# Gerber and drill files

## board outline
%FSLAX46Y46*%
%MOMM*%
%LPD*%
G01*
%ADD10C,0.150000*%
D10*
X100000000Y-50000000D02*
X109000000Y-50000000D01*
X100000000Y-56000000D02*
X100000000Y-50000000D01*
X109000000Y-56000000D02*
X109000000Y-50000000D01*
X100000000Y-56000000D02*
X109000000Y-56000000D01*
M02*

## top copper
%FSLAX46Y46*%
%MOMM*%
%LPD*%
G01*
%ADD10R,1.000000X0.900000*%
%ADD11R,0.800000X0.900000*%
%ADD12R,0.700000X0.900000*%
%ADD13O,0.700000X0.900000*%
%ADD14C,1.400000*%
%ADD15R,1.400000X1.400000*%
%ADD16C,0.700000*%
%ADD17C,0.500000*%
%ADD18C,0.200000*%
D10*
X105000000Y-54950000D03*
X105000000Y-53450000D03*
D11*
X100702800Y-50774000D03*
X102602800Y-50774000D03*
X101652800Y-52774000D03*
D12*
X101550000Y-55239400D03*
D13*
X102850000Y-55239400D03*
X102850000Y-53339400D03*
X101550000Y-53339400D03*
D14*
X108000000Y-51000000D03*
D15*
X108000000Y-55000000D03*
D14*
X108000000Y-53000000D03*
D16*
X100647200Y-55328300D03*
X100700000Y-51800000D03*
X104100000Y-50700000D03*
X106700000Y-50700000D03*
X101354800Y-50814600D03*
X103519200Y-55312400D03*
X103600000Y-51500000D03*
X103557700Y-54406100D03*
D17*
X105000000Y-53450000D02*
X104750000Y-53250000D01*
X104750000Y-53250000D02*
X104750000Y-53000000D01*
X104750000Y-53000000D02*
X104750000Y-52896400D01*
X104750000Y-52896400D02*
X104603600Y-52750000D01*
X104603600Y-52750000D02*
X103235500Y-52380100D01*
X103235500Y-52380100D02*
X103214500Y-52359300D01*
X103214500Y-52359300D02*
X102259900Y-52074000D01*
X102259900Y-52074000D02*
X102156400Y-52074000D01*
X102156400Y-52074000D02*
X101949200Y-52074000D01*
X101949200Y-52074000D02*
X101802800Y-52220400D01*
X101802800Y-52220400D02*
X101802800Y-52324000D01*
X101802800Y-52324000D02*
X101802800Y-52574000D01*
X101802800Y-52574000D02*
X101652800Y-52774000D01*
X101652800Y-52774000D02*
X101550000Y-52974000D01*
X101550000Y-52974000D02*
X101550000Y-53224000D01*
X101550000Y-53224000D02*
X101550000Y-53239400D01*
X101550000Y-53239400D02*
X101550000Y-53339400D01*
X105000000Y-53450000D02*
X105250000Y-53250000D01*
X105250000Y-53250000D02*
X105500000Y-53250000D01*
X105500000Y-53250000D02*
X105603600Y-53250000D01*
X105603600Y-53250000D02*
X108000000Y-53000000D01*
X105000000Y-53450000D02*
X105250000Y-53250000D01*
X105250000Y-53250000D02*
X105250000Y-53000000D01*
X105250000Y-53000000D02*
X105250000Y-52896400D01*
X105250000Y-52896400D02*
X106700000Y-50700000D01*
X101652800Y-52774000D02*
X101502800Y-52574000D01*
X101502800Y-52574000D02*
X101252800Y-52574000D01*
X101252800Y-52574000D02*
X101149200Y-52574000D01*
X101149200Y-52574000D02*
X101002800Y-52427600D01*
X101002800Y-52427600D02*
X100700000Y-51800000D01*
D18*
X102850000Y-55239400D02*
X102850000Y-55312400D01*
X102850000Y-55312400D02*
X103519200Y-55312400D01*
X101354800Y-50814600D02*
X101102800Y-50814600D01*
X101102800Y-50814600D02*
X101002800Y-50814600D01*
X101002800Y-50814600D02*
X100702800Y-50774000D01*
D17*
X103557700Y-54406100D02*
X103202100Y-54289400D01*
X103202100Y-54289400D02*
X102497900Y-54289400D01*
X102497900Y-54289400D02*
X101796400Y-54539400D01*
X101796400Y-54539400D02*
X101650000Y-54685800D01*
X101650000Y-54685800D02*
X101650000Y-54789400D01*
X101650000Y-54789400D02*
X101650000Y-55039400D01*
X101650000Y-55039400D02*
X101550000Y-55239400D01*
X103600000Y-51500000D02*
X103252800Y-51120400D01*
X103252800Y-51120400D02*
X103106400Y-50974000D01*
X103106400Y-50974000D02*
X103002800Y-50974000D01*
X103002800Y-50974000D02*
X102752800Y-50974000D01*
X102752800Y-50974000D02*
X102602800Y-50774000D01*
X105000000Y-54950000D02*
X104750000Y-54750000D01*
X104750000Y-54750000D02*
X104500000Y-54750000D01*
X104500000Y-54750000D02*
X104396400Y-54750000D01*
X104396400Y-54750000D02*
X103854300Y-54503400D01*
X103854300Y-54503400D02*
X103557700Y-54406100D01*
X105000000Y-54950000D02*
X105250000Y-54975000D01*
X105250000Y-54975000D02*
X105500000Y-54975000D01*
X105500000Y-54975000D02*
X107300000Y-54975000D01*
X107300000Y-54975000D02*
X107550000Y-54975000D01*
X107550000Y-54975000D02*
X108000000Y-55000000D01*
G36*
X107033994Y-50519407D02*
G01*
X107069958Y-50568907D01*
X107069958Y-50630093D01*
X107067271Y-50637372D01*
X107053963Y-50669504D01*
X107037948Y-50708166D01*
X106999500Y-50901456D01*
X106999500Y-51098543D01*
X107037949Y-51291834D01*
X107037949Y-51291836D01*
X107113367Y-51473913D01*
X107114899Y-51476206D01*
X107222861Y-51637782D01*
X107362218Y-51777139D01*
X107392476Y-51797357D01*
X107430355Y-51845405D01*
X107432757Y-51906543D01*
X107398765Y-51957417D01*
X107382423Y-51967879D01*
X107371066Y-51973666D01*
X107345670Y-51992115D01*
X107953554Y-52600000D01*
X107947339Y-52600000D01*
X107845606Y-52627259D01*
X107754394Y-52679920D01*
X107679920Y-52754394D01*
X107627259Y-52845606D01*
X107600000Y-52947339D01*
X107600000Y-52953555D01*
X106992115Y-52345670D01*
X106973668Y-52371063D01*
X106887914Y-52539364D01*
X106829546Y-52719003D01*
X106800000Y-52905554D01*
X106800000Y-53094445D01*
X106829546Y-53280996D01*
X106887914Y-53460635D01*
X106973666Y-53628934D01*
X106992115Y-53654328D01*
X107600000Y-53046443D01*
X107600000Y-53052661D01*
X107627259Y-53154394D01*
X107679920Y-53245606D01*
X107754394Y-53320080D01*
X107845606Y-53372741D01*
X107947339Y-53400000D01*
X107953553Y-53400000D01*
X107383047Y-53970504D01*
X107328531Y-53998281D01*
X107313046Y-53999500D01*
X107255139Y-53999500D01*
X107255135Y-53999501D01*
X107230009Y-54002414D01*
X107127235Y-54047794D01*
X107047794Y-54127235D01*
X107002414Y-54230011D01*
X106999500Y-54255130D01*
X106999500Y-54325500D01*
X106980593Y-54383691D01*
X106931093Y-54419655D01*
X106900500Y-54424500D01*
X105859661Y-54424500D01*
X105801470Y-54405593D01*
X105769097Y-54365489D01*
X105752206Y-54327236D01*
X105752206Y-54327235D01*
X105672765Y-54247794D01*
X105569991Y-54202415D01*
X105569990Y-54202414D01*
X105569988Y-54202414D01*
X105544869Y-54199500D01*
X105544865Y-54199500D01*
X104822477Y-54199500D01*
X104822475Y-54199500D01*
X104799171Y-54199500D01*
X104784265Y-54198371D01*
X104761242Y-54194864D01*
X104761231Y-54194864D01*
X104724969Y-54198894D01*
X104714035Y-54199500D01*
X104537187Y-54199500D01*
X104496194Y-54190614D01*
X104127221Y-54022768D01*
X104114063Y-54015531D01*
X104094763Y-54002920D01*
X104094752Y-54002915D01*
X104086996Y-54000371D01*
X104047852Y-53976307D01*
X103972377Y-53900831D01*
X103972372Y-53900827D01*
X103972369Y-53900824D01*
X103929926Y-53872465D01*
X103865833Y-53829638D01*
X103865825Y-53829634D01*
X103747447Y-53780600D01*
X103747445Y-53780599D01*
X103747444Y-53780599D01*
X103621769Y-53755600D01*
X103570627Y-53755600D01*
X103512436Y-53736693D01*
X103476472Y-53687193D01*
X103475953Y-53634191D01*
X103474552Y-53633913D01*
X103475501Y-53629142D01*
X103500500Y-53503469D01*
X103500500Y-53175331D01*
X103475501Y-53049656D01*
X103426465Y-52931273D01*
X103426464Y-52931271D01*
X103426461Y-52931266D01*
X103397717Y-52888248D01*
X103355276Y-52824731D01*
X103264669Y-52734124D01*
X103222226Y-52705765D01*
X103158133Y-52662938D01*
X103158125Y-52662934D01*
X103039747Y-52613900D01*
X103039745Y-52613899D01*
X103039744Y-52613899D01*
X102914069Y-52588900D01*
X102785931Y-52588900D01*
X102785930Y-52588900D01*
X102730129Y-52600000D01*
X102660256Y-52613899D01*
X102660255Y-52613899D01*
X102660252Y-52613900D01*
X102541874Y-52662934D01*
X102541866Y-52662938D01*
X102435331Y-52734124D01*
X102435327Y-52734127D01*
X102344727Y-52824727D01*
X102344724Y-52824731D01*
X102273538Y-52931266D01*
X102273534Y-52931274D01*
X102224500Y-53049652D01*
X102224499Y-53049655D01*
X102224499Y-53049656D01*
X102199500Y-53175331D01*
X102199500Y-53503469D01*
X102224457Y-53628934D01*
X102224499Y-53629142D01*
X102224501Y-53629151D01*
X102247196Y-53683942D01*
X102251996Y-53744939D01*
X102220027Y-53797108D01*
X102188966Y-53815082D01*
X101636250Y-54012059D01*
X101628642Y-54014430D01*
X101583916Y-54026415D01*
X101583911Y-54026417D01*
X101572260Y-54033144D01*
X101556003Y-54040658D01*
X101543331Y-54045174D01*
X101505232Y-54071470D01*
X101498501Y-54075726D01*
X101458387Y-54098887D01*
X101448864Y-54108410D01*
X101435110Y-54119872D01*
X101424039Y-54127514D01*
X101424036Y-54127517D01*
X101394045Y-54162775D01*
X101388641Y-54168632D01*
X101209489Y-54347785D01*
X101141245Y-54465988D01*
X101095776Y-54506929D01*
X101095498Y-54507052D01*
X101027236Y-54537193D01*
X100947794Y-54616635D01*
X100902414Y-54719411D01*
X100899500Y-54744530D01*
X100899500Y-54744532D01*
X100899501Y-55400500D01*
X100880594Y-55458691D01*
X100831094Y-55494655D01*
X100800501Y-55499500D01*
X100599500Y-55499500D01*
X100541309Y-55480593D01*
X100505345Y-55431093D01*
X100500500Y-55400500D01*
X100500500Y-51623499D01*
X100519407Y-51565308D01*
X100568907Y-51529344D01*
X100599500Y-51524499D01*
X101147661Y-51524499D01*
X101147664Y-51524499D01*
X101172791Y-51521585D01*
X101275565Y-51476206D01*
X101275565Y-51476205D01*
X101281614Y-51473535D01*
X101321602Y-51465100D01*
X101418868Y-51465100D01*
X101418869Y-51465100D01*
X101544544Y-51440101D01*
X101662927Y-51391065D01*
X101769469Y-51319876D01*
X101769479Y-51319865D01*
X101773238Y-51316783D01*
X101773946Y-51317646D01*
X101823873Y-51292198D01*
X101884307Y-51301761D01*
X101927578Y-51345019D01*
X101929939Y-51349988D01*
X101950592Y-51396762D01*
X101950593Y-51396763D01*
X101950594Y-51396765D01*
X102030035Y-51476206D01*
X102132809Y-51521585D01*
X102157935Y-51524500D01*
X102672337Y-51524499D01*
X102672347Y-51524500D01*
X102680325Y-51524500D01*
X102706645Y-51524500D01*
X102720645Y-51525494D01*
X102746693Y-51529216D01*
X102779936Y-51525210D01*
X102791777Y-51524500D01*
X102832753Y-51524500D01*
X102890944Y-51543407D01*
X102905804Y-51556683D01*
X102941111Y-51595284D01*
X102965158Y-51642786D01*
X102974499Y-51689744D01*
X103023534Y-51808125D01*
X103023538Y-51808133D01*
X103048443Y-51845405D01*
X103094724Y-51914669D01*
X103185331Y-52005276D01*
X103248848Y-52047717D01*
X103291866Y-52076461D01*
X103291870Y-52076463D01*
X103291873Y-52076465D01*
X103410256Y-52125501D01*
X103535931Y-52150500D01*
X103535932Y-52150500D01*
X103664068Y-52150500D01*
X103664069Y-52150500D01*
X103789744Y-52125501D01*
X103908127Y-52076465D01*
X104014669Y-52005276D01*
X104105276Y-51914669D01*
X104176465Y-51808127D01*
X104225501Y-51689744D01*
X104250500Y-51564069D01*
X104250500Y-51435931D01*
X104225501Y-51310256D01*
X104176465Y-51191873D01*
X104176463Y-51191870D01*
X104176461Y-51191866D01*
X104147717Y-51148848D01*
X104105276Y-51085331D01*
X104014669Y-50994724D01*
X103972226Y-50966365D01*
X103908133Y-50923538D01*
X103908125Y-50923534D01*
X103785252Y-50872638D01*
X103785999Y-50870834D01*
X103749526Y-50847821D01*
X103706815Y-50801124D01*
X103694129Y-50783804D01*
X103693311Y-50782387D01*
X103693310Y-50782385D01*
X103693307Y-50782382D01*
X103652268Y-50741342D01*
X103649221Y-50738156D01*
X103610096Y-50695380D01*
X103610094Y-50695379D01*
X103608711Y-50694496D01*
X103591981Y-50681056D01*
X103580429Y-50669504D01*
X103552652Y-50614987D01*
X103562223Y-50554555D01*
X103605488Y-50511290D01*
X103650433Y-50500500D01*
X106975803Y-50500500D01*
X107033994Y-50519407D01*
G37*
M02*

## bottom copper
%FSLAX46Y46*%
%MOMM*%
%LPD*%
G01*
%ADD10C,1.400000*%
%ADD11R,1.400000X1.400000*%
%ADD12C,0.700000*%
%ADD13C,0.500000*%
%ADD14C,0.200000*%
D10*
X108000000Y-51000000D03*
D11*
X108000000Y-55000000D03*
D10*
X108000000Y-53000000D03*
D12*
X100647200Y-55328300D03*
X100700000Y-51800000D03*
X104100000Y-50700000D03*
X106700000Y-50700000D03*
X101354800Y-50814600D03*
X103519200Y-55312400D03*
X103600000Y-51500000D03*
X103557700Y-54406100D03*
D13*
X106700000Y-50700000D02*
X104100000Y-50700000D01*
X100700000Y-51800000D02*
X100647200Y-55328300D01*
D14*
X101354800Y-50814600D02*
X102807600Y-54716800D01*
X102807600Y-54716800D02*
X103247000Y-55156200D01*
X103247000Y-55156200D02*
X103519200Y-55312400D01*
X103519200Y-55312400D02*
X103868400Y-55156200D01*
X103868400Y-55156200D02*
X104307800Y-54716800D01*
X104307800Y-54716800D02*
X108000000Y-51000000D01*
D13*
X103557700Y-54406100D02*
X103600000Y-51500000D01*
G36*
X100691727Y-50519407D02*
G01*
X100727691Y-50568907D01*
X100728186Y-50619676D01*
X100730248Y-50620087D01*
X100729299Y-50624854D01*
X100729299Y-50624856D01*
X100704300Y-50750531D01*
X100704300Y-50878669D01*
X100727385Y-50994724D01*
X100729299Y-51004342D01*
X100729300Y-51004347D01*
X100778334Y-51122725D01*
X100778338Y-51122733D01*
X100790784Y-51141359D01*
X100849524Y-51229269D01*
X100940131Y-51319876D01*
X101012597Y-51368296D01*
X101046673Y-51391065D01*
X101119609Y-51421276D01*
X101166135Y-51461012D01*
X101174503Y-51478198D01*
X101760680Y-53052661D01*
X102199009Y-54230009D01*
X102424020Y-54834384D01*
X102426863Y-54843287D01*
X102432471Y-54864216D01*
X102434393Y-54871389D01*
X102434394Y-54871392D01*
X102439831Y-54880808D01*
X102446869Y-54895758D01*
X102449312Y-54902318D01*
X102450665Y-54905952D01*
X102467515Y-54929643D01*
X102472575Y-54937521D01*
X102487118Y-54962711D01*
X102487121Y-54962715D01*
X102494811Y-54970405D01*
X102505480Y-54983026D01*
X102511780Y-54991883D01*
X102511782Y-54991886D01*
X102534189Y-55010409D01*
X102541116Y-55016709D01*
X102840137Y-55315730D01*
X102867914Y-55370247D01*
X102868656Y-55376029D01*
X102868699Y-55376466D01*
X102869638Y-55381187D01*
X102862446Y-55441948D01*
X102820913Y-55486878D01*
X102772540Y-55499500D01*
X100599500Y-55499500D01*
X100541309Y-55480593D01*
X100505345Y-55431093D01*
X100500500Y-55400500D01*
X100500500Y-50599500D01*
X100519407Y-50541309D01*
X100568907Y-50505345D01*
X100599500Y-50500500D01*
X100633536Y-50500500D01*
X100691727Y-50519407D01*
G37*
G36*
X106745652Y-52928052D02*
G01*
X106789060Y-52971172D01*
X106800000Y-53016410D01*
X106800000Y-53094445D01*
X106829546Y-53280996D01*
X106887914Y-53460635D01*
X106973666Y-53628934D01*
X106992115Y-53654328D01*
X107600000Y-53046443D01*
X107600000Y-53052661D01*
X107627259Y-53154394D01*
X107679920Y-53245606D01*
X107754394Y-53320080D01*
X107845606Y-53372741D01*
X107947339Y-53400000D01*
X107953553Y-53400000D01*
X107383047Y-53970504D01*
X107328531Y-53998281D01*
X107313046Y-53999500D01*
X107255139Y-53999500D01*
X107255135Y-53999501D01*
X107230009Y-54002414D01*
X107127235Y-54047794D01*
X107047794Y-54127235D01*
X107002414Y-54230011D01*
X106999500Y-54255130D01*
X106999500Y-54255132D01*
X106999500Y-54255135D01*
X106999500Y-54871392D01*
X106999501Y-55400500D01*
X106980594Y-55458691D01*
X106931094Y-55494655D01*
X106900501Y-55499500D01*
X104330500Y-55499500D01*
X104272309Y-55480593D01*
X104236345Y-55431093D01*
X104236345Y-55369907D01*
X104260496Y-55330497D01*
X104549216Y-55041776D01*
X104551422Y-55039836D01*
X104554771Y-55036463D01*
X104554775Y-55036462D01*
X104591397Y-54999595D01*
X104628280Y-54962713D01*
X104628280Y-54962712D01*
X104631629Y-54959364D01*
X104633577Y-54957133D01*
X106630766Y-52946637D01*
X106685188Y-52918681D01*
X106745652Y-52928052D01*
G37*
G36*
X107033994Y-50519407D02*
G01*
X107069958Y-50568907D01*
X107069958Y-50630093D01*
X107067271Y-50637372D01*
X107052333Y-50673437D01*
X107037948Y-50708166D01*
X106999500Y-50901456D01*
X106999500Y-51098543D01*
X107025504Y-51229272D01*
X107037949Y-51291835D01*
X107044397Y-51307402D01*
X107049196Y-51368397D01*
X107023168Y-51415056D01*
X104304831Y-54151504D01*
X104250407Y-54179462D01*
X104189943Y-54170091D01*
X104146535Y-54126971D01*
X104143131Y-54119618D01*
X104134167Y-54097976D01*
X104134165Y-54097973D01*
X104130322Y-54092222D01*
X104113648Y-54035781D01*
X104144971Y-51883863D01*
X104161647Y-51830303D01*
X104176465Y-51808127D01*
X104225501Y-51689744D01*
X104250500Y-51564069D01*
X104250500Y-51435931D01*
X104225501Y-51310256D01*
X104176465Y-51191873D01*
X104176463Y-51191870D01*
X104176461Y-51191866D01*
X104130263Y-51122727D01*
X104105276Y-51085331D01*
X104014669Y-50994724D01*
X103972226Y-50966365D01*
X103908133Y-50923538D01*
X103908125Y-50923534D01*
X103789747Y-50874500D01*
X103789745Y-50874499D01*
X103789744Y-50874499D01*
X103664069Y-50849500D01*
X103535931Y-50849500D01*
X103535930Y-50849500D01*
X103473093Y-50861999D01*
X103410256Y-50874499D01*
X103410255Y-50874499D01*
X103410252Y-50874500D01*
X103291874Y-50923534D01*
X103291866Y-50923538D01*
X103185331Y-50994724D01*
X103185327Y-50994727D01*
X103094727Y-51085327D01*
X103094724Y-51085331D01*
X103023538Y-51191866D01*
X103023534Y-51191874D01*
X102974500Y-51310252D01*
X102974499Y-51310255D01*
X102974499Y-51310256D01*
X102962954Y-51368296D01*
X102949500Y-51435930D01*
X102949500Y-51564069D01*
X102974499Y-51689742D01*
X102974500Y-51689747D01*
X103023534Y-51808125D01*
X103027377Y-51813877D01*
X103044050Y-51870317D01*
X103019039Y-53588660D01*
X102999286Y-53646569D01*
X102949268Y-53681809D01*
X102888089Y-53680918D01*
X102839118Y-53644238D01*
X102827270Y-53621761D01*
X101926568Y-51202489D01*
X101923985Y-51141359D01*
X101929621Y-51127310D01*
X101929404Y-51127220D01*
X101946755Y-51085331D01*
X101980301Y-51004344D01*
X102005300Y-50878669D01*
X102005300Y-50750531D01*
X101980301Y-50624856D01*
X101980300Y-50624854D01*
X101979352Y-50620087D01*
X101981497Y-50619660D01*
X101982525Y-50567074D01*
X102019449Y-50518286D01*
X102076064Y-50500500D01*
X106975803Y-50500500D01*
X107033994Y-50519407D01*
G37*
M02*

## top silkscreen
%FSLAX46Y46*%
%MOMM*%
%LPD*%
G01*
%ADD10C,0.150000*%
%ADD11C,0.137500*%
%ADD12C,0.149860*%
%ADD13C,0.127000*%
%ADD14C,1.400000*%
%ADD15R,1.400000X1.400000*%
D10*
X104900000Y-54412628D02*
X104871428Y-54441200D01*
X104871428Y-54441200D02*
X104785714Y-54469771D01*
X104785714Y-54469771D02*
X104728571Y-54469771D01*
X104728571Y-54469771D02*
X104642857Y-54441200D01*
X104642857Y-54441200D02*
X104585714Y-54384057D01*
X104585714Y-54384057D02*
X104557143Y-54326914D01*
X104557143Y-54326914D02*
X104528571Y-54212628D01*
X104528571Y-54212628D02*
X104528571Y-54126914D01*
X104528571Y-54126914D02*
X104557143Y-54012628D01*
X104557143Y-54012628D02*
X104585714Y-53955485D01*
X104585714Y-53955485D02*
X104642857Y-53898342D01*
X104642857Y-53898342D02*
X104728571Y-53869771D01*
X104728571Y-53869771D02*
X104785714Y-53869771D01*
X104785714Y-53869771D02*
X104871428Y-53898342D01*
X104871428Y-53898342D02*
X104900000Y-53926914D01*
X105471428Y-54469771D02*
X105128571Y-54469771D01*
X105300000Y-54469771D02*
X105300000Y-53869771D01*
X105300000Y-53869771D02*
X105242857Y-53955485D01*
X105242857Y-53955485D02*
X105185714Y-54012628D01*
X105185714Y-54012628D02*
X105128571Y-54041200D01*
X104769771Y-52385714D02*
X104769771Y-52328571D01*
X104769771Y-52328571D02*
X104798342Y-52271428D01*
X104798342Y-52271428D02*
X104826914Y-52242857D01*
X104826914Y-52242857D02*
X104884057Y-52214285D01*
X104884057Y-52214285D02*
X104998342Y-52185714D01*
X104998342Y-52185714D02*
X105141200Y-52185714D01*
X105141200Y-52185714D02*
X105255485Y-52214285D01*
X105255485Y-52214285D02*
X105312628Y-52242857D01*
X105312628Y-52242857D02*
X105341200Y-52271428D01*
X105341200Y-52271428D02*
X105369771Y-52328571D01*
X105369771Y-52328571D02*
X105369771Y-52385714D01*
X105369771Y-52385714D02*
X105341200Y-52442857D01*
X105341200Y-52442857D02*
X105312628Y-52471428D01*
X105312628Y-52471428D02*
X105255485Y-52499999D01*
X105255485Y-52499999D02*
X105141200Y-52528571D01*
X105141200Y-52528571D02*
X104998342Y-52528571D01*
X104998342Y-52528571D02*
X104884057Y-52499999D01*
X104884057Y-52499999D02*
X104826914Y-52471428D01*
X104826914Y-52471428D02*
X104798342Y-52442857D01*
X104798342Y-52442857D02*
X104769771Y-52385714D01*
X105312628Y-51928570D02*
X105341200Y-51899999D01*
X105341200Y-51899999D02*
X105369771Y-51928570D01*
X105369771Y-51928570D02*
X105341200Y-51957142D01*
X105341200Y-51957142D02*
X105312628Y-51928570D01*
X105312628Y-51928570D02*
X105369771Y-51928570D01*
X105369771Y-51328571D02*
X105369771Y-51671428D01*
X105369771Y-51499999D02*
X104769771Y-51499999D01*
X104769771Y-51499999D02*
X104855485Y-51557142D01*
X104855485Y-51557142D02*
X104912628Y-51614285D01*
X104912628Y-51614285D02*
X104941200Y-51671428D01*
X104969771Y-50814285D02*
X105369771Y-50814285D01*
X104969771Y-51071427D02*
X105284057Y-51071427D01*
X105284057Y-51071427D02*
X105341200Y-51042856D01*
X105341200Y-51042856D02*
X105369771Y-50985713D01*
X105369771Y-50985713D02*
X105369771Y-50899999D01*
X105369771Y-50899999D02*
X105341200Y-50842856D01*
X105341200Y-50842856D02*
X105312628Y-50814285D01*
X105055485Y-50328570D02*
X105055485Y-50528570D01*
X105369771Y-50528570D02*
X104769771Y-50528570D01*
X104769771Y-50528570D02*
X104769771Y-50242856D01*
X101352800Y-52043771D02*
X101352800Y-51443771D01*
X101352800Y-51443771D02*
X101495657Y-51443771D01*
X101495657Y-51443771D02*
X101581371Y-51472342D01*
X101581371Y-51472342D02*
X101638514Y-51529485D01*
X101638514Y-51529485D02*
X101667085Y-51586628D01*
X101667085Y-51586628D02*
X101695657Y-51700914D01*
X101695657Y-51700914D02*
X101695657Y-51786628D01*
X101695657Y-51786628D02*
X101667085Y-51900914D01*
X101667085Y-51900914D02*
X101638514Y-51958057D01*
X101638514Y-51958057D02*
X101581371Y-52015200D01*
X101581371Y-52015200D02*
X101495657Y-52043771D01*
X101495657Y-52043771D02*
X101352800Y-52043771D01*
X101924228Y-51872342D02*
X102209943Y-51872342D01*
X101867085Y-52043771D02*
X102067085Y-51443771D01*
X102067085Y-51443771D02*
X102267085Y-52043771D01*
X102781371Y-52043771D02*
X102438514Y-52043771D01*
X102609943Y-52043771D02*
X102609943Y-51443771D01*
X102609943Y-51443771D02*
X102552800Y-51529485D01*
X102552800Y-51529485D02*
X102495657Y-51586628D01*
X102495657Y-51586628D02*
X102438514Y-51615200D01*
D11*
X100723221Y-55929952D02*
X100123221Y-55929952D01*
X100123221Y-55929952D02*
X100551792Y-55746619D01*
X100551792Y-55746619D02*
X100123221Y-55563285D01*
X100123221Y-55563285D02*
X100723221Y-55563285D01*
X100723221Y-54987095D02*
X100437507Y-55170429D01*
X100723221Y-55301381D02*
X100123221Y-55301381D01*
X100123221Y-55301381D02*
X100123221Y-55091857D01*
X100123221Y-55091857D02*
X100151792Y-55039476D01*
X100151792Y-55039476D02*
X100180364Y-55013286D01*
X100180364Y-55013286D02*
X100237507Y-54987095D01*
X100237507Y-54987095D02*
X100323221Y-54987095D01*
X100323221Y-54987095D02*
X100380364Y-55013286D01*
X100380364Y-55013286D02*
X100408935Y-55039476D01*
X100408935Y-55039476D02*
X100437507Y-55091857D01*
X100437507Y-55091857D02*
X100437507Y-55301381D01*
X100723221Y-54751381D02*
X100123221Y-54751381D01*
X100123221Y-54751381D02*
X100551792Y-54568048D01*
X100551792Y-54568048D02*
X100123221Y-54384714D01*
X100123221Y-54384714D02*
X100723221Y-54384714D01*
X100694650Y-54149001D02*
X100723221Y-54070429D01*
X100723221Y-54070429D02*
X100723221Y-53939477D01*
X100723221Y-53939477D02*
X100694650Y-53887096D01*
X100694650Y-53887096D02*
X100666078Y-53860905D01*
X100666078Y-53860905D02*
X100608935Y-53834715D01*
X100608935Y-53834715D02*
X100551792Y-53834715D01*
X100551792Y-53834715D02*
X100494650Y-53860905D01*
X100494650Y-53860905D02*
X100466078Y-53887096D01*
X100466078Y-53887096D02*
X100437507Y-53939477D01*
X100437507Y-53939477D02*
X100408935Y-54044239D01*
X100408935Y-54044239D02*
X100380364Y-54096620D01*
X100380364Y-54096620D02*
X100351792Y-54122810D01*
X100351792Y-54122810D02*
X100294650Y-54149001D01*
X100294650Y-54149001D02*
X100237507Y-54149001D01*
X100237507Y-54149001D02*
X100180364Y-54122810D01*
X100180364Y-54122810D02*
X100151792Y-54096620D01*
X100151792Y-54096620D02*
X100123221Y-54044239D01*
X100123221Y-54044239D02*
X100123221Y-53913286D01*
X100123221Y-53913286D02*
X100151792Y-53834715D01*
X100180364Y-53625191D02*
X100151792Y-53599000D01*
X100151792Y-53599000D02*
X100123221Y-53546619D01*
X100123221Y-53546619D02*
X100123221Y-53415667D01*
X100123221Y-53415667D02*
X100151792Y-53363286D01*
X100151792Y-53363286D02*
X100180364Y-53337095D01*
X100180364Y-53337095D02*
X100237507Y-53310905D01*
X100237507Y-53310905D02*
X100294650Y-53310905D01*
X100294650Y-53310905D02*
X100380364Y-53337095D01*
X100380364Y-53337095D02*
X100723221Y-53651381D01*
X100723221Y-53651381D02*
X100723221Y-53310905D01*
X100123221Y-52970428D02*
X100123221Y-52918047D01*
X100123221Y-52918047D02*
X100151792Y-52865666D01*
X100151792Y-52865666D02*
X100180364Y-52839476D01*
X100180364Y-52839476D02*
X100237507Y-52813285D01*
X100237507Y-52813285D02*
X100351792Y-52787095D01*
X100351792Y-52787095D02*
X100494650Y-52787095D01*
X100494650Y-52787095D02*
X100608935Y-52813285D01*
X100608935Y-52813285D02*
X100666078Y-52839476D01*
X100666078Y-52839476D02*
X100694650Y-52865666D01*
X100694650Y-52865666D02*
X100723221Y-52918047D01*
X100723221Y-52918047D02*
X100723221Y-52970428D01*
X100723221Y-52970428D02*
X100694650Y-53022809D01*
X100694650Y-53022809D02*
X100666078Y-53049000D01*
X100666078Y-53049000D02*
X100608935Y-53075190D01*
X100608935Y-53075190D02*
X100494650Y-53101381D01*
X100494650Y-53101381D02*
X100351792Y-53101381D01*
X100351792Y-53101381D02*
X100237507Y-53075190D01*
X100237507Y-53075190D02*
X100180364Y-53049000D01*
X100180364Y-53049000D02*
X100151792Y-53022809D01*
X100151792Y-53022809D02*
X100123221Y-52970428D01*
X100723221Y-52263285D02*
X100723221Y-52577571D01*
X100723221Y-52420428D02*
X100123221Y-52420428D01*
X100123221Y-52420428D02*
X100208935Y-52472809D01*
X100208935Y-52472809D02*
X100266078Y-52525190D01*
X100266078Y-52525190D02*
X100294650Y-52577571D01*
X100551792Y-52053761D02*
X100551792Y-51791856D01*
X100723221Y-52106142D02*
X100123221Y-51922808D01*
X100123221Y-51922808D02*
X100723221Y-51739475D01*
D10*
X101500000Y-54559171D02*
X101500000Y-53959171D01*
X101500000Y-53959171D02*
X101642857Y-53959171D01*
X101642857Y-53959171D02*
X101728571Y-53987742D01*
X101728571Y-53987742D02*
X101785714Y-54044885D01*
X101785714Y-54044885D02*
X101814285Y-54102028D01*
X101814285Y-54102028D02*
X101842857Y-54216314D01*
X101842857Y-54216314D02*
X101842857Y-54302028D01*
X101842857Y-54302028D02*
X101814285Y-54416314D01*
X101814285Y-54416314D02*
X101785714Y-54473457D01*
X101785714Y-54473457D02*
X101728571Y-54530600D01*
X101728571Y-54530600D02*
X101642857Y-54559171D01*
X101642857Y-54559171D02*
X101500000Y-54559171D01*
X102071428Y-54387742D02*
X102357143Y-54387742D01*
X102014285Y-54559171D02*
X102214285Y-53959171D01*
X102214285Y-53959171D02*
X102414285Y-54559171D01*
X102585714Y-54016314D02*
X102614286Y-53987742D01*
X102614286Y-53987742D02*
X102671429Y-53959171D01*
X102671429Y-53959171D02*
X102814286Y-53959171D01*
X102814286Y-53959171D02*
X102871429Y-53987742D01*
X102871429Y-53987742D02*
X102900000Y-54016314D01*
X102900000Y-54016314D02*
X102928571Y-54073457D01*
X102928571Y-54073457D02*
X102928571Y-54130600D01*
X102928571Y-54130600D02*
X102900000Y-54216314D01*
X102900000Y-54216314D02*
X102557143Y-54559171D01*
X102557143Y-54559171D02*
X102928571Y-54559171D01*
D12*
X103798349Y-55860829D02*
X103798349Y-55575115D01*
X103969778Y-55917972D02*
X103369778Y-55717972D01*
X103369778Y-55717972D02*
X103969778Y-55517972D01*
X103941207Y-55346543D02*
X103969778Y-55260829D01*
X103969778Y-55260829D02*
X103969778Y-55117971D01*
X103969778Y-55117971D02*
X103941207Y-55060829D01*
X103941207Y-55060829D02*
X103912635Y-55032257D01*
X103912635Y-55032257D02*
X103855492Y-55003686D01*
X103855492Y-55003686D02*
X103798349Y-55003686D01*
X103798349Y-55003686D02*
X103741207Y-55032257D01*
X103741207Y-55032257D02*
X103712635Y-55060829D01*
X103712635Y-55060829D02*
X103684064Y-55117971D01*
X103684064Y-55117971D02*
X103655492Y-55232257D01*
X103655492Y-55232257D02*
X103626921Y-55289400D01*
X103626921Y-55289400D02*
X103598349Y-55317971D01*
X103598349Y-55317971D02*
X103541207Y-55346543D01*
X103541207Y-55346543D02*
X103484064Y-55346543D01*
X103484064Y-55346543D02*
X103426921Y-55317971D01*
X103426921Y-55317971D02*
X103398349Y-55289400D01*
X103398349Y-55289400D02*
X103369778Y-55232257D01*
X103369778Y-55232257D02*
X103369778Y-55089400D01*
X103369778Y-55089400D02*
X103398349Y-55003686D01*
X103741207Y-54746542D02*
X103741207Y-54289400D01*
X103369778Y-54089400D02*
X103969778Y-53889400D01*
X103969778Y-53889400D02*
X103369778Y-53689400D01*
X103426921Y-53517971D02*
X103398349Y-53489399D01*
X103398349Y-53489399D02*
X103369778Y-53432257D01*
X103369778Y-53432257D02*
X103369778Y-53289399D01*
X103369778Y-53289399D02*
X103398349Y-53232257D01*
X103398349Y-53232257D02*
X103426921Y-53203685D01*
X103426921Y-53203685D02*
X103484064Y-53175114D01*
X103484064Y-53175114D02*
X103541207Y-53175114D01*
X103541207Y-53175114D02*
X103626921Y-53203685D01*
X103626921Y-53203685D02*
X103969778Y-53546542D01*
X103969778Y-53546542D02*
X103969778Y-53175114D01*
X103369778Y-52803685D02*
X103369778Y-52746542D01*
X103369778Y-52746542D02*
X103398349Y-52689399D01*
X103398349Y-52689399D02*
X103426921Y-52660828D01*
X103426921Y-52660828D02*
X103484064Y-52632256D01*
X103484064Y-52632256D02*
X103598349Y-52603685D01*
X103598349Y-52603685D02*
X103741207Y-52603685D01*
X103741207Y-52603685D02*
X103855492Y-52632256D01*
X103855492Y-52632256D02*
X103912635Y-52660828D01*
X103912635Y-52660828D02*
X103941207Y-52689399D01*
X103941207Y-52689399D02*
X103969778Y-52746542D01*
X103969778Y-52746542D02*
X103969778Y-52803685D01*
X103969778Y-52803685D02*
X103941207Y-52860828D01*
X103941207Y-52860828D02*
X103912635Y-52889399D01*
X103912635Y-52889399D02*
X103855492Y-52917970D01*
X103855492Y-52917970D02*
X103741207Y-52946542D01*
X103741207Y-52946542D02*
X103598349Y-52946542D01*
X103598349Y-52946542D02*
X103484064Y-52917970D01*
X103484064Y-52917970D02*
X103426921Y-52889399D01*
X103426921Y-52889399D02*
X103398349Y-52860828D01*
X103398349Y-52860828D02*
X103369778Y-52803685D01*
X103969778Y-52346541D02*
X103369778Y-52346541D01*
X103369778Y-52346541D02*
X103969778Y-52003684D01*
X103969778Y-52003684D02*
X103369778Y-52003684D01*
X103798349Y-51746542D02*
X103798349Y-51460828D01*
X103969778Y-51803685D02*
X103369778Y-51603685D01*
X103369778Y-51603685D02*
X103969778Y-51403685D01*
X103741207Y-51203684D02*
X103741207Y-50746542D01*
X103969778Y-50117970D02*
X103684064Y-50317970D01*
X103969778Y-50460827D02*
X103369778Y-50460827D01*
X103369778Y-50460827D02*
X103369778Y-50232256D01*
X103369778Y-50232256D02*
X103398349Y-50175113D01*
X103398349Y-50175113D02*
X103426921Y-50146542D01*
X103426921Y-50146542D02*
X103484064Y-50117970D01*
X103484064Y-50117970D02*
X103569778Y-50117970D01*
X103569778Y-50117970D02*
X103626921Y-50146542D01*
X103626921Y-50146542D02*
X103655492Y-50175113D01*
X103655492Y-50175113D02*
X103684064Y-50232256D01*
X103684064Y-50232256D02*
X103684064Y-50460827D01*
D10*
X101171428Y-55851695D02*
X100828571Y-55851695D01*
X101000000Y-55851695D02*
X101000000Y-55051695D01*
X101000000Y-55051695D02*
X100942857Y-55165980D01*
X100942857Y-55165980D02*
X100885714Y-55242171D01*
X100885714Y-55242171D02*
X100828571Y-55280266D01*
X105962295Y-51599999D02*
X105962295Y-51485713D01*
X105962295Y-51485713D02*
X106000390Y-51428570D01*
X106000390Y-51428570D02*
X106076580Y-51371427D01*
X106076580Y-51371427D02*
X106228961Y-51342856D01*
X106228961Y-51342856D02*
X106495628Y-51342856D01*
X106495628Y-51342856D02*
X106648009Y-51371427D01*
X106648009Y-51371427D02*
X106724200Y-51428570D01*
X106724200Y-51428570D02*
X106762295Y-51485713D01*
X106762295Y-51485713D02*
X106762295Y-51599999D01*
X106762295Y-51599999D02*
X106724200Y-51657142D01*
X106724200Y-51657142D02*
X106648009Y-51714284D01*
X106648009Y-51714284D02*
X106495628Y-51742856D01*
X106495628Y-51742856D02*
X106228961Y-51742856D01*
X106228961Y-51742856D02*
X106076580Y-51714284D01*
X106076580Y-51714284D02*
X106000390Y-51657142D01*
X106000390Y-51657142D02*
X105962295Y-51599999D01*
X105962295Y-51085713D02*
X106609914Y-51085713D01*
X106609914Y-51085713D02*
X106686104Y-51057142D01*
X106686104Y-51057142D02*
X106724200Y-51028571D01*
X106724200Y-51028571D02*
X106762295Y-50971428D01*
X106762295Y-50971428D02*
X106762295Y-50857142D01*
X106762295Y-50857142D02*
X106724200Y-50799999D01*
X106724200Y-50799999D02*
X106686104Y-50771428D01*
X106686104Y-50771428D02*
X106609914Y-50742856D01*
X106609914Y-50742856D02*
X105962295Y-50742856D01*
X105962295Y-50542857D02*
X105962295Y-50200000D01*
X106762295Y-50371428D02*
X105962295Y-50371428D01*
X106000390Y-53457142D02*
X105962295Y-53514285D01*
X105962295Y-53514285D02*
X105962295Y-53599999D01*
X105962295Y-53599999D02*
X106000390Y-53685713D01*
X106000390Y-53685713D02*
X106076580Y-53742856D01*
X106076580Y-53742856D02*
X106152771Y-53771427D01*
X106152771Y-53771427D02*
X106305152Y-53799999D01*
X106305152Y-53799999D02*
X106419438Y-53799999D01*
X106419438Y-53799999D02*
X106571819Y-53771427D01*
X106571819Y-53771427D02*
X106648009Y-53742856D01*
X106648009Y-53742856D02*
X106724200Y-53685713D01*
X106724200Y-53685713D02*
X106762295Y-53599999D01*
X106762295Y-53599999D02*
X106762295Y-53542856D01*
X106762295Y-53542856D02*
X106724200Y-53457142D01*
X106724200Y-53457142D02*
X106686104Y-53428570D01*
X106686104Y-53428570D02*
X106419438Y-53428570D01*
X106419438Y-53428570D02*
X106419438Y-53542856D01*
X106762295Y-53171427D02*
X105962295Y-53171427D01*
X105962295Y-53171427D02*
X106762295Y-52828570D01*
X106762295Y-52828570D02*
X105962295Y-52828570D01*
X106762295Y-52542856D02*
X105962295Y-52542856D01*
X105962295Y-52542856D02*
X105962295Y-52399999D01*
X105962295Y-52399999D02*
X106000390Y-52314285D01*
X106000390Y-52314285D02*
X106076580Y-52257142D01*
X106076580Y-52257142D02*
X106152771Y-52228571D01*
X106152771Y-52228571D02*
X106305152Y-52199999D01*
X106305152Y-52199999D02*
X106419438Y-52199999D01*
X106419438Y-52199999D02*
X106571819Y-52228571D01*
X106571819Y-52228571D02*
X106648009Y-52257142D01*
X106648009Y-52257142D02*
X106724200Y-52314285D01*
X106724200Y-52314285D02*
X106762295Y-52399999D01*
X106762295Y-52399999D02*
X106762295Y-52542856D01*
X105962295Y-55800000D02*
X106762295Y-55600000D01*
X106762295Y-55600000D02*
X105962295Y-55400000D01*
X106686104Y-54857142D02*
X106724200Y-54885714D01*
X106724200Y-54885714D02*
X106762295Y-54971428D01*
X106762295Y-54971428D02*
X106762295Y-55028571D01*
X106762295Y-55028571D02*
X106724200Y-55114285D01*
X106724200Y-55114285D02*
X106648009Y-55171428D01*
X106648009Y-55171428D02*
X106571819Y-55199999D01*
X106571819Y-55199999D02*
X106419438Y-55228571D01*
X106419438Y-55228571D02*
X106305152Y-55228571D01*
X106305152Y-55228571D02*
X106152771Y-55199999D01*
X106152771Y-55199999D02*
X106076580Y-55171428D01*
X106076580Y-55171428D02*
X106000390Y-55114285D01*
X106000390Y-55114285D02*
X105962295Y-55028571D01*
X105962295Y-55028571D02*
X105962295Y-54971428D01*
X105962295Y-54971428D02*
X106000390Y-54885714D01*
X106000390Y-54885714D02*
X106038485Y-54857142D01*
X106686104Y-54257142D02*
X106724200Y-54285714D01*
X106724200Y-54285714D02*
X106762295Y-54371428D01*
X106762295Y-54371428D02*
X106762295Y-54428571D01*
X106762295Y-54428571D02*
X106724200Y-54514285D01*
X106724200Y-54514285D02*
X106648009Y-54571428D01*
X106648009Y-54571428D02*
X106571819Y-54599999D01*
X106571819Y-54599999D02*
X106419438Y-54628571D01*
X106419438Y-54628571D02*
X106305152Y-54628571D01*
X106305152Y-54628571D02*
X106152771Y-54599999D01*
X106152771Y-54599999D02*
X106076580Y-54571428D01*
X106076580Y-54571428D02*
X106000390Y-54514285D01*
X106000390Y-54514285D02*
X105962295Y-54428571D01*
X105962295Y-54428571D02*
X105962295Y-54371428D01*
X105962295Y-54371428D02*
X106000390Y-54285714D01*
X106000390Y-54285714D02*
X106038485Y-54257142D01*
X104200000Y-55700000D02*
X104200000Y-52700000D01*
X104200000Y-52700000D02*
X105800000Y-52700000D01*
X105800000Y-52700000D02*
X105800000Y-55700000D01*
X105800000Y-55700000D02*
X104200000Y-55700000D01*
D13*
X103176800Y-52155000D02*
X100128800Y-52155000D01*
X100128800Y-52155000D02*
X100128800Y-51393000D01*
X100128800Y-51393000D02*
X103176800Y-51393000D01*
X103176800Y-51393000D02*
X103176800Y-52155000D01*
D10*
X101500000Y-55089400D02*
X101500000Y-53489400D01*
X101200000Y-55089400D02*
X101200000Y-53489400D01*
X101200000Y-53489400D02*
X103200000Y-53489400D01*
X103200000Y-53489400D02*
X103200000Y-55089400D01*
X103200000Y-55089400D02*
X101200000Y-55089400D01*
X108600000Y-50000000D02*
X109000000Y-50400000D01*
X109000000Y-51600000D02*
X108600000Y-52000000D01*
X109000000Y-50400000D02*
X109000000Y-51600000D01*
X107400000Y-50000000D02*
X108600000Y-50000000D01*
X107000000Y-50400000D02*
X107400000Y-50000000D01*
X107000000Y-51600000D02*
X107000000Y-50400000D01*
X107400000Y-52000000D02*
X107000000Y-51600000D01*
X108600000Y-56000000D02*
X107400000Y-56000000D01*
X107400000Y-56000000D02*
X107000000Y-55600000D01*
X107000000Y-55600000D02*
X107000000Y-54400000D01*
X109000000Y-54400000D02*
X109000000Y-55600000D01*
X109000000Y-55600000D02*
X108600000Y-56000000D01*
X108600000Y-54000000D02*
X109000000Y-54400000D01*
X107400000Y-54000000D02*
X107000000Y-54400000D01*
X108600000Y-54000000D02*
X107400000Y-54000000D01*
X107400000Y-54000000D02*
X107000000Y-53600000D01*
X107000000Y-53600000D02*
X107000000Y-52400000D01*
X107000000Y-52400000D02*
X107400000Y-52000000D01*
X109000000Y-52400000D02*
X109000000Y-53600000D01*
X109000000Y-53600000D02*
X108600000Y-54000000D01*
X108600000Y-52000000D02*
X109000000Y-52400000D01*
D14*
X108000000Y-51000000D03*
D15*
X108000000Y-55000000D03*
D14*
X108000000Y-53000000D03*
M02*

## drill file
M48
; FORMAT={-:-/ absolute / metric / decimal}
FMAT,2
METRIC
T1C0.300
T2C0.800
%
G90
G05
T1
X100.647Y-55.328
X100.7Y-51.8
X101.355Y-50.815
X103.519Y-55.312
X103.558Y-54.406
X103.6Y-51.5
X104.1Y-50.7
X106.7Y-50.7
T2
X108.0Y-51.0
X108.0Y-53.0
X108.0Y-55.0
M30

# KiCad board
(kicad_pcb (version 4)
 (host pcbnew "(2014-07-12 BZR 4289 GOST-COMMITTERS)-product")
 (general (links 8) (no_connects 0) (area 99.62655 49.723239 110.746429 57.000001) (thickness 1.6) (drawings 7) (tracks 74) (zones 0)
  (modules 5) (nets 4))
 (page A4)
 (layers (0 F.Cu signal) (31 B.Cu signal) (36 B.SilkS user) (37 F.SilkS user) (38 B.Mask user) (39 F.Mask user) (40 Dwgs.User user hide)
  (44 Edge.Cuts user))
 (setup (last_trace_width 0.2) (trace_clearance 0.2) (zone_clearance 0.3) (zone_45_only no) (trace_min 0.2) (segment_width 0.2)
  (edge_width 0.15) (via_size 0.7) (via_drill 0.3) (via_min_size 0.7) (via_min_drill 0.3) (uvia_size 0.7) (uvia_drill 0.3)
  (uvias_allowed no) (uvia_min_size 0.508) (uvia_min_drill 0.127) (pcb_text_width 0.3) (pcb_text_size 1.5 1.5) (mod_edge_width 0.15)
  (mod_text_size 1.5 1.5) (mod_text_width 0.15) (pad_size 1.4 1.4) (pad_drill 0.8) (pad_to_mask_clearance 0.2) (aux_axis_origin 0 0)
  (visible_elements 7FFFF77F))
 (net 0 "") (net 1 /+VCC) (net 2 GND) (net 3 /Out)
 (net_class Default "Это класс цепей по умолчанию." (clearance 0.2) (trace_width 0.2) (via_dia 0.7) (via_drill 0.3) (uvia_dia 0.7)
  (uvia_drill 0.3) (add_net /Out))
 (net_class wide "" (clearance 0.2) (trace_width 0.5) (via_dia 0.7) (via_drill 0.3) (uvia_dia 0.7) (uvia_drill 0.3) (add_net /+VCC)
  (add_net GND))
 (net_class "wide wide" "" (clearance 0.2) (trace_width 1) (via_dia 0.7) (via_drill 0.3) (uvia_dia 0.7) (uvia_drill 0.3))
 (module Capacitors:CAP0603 (layer F.Cu) (at 105 54.2 90)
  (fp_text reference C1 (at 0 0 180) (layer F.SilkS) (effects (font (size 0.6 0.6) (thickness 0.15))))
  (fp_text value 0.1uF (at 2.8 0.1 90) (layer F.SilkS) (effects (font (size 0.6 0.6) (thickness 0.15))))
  (fp_line (start -1.5 -0.8) (end 1.5 -0.8) (layer F.SilkS) (width 0.15))
  (fp_line (start 1.5 -0.8) (end 1.5 0.8) (layer F.SilkS) (width 0.15))
  (fp_line (start 1.5 0.8) (end -1.5 0.8) (layer F.SilkS) (width 0.15))
  (fp_line (start -1.5 0.8) (end -1.5 -0.8) (layer F.SilkS) (width 0.15))
  (pad 1 smd rect (at -0.75 0 90) (size 0.9 1) (layers F.Cu F.Mask) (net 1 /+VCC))
  (pad 2 smd rect (at 0.75 0 90) (size 0.9 1) (layers F.Cu F.Mask) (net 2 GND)))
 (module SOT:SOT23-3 (layer F.Cu) (at 101.6528 51.774 180)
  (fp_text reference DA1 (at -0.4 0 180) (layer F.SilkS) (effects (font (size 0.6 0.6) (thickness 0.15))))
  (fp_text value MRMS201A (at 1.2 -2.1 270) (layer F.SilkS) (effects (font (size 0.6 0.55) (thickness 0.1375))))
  (fp_line (start -1.524 -0.381) (end 1.524 -0.381) (layer F.SilkS) (width 0.127))
  (fp_line (start 1.524 -0.381) (end 1.524 0.381) (layer F.SilkS) (width 0.127))
  (fp_line (start 1.524 0.381) (end -1.524 0.381) (layer F.SilkS) (width 0.127))
  (fp_line (start -1.524 0.381) (end -1.524 -0.381) (layer F.SilkS) (width 0.127))
  (pad 2 smd rect (at 0.95 1 180) (size 0.8 0.9) (layers F.Cu F.Mask) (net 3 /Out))
  (pad 1 smd rect (at -0.95 1 180) (size 0.8 0.9) (layers F.Cu F.Mask) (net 1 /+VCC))
  (pad 3 smd rect (at 0 -1 180) (size 0.8 0.9) (layers F.Cu F.Mask) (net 2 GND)))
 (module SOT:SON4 (layer F.Cu) (at 102.2 54.2894 90)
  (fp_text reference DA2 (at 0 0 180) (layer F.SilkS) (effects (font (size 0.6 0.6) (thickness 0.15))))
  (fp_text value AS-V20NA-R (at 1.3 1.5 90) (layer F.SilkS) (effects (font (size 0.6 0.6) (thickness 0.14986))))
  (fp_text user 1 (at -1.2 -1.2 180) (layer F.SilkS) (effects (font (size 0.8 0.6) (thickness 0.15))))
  (fp_line (start -0.8 -0.7) (end 0.8 -0.7) (layer F.SilkS) (width 0.15))
  (fp_line (start -0.8 -1) (end 0.8 -1) (layer F.SilkS) (width 0.15))
  (fp_line (start 0.8 -1) (end 0.8 1) (layer F.SilkS) (width 0.15))
  (fp_line (start 0.8 1) (end -0.8 1) (layer F.SilkS) (width 0.15))
  (fp_line (start -0.8 1) (end -0.8 -1) (layer F.SilkS) (width 0.15))
  (pad 1 smd rect (at -0.95 -0.65 90) (size 0.9 0.7) (layers F.Cu F.Mask) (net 1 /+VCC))
  (pad 2 smd oval (at -0.95 0.65 90) (size 0.9 0.7) (layers F.Cu F.Mask) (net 3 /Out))
  (pad 3 smd oval (at 0.95 0.65 90) (size 0.9 0.7) (layers F.Cu F.Mask))
  (pad 4 smd oval (at 0.95 -0.65 90) (size 0.9 0.7) (layers F.Cu F.Mask) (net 2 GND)))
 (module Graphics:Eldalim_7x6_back (layer B.Cu) (at 103.5 52.9)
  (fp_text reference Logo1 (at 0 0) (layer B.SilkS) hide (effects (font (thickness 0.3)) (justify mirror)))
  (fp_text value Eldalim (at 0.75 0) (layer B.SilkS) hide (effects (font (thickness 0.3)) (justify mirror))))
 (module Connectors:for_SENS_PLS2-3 (layer F.Cu) (at 108 55 90)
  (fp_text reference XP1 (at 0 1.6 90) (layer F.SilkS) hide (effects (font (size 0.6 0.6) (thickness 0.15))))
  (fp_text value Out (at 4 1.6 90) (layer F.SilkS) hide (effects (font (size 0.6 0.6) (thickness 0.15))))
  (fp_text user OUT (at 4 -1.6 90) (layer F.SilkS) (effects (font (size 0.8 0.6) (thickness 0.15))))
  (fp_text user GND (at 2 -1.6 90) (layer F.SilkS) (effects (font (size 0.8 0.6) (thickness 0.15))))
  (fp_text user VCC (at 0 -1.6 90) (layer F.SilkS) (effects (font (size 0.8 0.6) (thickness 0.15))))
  (fp_line (start 5 0.6) (end 4.6 1) (layer F.SilkS) (width 0.15))
  (fp_line (start 3.4 1) (end 3 0.6) (layer F.SilkS) (width 0.15))
  (fp_line (start 4.6 1) (end 3.4 1) (layer F.SilkS) (width 0.15))
  (fp_line (start 5 -0.6) (end 5 0.6) (layer F.SilkS) (width 0.15))
  (fp_line (start 4.6 -1) (end 5 -0.6) (layer F.SilkS) (width 0.15))
  (fp_line (start 3.4 -1) (end 4.6 -1) (layer F.SilkS) (width 0.15))
  (fp_line (start 3 -0.6) (end 3.4 -1) (layer F.SilkS) (width 0.15))
  (fp_line (start -1 0.6) (end -1 -0.6) (layer F.SilkS) (width 0.15))
  (fp_line (start -1 -0.6) (end -0.6 -1) (layer F.SilkS) (width 0.15))
  (fp_line (start -0.6 -1) (end 0.6 -1) (layer F.SilkS) (width 0.15))
  (fp_line (start 0.6 1) (end -0.6 1) (layer F.SilkS) (width 0.15))
  (fp_line (start -0.6 1) (end -1 0.6) (layer F.SilkS) (width 0.15))
  (fp_line (start 1 0.6) (end 0.6 1) (layer F.SilkS) (width 0.15))
  (fp_line (start 1 -0.6) (end 0.6 -1) (layer F.SilkS) (width 0.15))
  (fp_line (start 1 0.6) (end 1 -0.6) (layer F.SilkS) (width 0.15))
  (fp_line (start 1 -0.6) (end 1.4 -1) (layer F.SilkS) (width 0.15))
  (fp_line (start 1.4 -1) (end 2.6 -1) (layer F.SilkS) (width 0.15))
  (fp_line (start 2.6 -1) (end 3 -0.6) (layer F.SilkS) (width 0.15))
  (fp_line (start 2.6 1) (end 1.4 1) (layer F.SilkS) (width 0.15))
  (fp_line (start 1.4 1) (end 1 0.6) (layer F.SilkS) (width 0.15))
  (fp_line (start 3 0.6) (end 2.6 1) (layer F.SilkS) (width 0.15))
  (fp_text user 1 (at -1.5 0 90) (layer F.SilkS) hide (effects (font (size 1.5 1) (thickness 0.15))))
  (pad 3 thru_hole circle (at 4 0 90) (size 1.4 1.4) (drill 0.8) (layers *.Cu *.Mask F.SilkS) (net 3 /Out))
  (pad 1 thru_hole rect (at 0 0 90) (size 1.4 1.4) (drill 0.8) (layers *.Cu *.Mask F.SilkS) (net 1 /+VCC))
  (pad 2 thru_hole circle (at 2 0 90) (size 1.4 1.4) (drill 0.8) (layers *.Cu *.Mask F.SilkS) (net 2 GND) (zone_connect 1)))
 (gr_line (start 100 50) (end 109 50) (angle 90) (layer Edge.Cuts) (width 0.15))
 (gr_line (start 100 56) (end 100 50) (angle 90) (layer Edge.Cuts) (width 0.15))
 (gr_line (start 109 56) (end 109 50) (angle 90) (layer Edge.Cuts) (width 0.15))
 (gr_line (start 100 56) (end 109 56) (angle 90) (layer Edge.Cuts) (width 0.15))
 (segment (start 105 53.45) (end 104.75 53.25) (width 0.5) (layer F.Cu) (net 2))
 (segment (start 104.75 53.25) (end 104.75 53) (width 0.5) (layer F.Cu) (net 2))
 (segment (start 104.75 53) (end 104.75 52.8964) (width 0.5) (layer F.Cu) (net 2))
 (segment (start 104.75 52.8964) (end 104.6036 52.75) (width 0.5) (layer F.Cu) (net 2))
 (segment (start 104.6036 52.75) (end 103.2355 52.3801) (width 0.5) (layer F.Cu) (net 2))
 (segment (start 103.2355 52.3801) (end 103.2145 52.3593) (width 0.5) (layer F.Cu) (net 2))
 (segment (start 103.2145 52.3593) (end 102.2599 52.074) (width 0.5) (layer F.Cu) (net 2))
 (segment (start 102.2599 52.074) (end 102.1564 52.074) (width 0.5) (layer F.Cu) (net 2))
 (segment (start 102.1564 52.074) (end 101.9492 52.074) (width 0.5) (layer F.Cu) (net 2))
 (segment (start 101.9492 52.074) (end 101.8028 52.2204) (width 0.5) (layer F.Cu) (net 2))
 (segment (start 101.8028 52.2204) (end 101.8028 52.324) (width 0.5) (layer F.Cu) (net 2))
 (segment (start 101.8028 52.324) (end 101.8028 52.574) (width 0.5) (layer F.Cu) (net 2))
 (segment (start 101.8028 52.574) (end 101.6528 52.774) (width 0.5) (layer F.Cu) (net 2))
 (segment (start 101.6528 52.774) (end 101.55 52.974) (width 0.5) (layer F.Cu) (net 2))
 (segment (start 101.55 52.974) (end 101.55 53.224) (width 0.5) (layer F.Cu) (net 2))
 (segment (start 101.55 53.224) (end 101.55 53.2394) (width 0.5) (layer F.Cu) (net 2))
 (segment (start 101.55 53.2394) (end 101.55 53.3394) (width 0.5) (layer F.Cu) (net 2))
 (segment (start 105 53.45) (end 105.25 53.25) (width 0.5) (layer F.Cu) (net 2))
 (segment (start 105.25 53.25) (end 105.5 53.25) (width 0.5) (layer F.Cu) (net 2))
 (segment (start 105.5 53.25) (end 105.6036 53.25) (width 0.5) (layer F.Cu) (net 2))
 (segment (start 105.6036 53.25) (end 108 53) (width 0.5) (layer F.Cu) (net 2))
 (segment (start 105 53.45) (end 105.25 53.25) (width 0.5) (layer F.Cu) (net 2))
 (segment (start 105.25 53.25) (end 105.25 53) (width 0.5) (layer F.Cu) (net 2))
 (segment (start 105.25 53) (end 105.25 52.8964) (width 0.5) (layer F.Cu) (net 2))
 (segment (start 105.25 52.8964) (end 106.7 50.7) (width 0.5) (layer F.Cu) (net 2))
 (segment (start 101.6528 52.774) (end 101.5028 52.574) (width 0.5) (layer F.Cu) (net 2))
 (segment (start 101.5028 52.574) (end 101.2528 52.574) (width 0.5) (layer F.Cu) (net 2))
 (segment (start 101.2528 52.574) (end 101.1492 52.574) (width 0.5) (layer F.Cu) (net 2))
 (segment (start 101.1492 52.574) (end 101.0028 52.4276) (width 0.5) (layer F.Cu) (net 2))
 (segment (start 101.0028 52.4276) (end 100.7 51.8) (width 0.5) (layer F.Cu) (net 2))
 (segment (start 106.7 50.7) (end 104.1 50.7) (width 0.5) (layer B.Cu) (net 2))
 (segment (start 100.7 51.8) (end 100.6472 55.3283) (width 0.5) (layer B.Cu) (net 2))
 (via (at 100.6472 55.3283) (size 0.7) (layers F.Cu B.Cu) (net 2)) (via (at 100.7 51.8) (size 0.7) (layers F.Cu B.Cu) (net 2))
 (via (at 104.1 50.7) (size 0.7) (layers F.Cu B.Cu) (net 2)) (via (at 106.7 50.7) (size 0.7) (layers F.Cu B.Cu) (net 2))
 (segment (start 102.85 55.2394) (end 102.85 55.3124) (width 0.2) (layer F.Cu) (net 3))
 (segment (start 102.85 55.3124) (end 103.5192 55.3124) (width 0.2) (layer F.Cu) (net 3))
 (segment (start 101.3548 50.8146) (end 101.1028 50.8146) (width 0.2) (layer F.Cu) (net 3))
 (segment (start 101.1028 50.8146) (end 101.0028 50.8146) (width 0.2) (layer F.Cu) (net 3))
 (segment (start 101.0028 50.8146) (end 100.7028 50.774) (width 0.2) (layer F.Cu) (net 3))
 (segment (start 101.3548 50.8146) (end 102.8076 54.7168) (width 0.2) (layer B.Cu) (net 3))
 (segment (start 102.8076 54.7168) (end 103.247 55.1562) (width 0.2) (layer B.Cu) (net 3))
 (segment (start 103.247 55.1562) (end 103.5192 55.3124) (width 0.2) (layer B.Cu) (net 3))
 (segment (start 103.5192 55.3124) (end 103.8684 55.1562) (width 0.2) (layer B.Cu) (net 3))
 (segment (start 103.8684 55.1562) (end 104.3078 54.7168) (width 0.2) (layer B.Cu) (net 3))
 (segment (start 104.3078 54.7168) (end 108 51) (width 0.2) (layer B.Cu) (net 3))
 (via (at 101.3548 50.8146) (size 0.7) (layers F.Cu B.Cu) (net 3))
 (via (at 103.5192 55.3124) (size 0.7) (layers F.Cu B.Cu) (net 3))
 (segment (start 103.5577 54.4061) (end 103.2021 54.2894) (width 0.5) (layer F.Cu) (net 1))
 (segment (start 103.2021 54.2894) (end 102.4979 54.2894) (width 0.5) (layer F.Cu) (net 1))
 (segment (start 102.4979 54.2894) (end 101.7964 54.5394) (width 0.5) (layer F.Cu) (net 1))
 (segment (start 101.7964 54.5394) (end 101.65 54.6858) (width 0.5) (layer F.Cu) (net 1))
 (segment (start 101.65 54.6858) (end 101.65 54.7894) (width 0.5) (layer F.Cu) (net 1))
 (segment (start 101.65 54.7894) (end 101.65 55.0394) (width 0.5) (layer F.Cu) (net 1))
 (segment (start 101.65 55.0394) (end 101.55 55.2394) (width 0.5) (layer F.Cu) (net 1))
 (segment (start 103.6 51.5) (end 103.2528 51.1204) (width 0.5) (layer F.Cu) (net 1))
 (segment (start 103.2528 51.1204) (end 103.1064 50.974) (width 0.5) (layer F.Cu) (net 1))
 (segment (start 103.1064 50.974) (end 103.0028 50.974) (width 0.5) (layer F.Cu) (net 1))
 (segment (start 103.0028 50.974) (end 102.7528 50.974) (width 0.5) (layer F.Cu) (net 1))
 (segment (start 102.7528 50.974) (end 102.6028 50.774) (width 0.5) (layer F.Cu) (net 1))
 (segment (start 105 54.95) (end 104.75 54.75) (width 0.5) (layer F.Cu) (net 1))
 (segment (start 104.75 54.75) (end 104.5 54.75) (width 0.5) (layer F.Cu) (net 1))
 (segment (start 104.5 54.75) (end 104.3964 54.75) (width 0.5) (layer F.Cu) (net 1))
 (segment (start 104.3964 54.75) (end 103.8543 54.5034) (width 0.5) (layer F.Cu) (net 1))
 (segment (start 103.8543 54.5034) (end 103.5577 54.4061) (width 0.5) (layer F.Cu) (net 1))
 (segment (start 105 54.95) (end 105.25 54.975) (width 0.5) (layer F.Cu) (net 1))
 (segment (start 105.25 54.975) (end 105.5 54.975) (width 0.5) (layer F.Cu) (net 1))
 (segment (start 105.5 54.975) (end 107.3 54.975) (width 0.5) (layer F.Cu) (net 1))
 (segment (start 107.3 54.975) (end 107.55 54.975) (width 0.5) (layer F.Cu) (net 1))
 (segment (start 107.55 54.975) (end 108 55) (width 0.5) (layer F.Cu) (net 1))
 (segment (start 103.5577 54.4061) (end 103.6 51.5) (width 0.5) (layer B.Cu) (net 1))
 (via (at 103.6 51.5) (size 0.7) (layers F.Cu B.Cu) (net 1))
 (via (at 103.5577 54.4061) (size 0.7) (layers F.Cu B.Cu) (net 1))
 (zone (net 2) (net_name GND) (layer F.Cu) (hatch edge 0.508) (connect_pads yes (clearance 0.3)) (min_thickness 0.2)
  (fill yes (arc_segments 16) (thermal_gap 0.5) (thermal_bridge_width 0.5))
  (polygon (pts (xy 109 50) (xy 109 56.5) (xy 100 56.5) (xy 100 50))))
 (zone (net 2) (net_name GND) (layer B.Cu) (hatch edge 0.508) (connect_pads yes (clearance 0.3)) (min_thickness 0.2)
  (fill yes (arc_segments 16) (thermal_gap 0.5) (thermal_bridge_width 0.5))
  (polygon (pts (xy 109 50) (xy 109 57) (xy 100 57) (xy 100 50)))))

